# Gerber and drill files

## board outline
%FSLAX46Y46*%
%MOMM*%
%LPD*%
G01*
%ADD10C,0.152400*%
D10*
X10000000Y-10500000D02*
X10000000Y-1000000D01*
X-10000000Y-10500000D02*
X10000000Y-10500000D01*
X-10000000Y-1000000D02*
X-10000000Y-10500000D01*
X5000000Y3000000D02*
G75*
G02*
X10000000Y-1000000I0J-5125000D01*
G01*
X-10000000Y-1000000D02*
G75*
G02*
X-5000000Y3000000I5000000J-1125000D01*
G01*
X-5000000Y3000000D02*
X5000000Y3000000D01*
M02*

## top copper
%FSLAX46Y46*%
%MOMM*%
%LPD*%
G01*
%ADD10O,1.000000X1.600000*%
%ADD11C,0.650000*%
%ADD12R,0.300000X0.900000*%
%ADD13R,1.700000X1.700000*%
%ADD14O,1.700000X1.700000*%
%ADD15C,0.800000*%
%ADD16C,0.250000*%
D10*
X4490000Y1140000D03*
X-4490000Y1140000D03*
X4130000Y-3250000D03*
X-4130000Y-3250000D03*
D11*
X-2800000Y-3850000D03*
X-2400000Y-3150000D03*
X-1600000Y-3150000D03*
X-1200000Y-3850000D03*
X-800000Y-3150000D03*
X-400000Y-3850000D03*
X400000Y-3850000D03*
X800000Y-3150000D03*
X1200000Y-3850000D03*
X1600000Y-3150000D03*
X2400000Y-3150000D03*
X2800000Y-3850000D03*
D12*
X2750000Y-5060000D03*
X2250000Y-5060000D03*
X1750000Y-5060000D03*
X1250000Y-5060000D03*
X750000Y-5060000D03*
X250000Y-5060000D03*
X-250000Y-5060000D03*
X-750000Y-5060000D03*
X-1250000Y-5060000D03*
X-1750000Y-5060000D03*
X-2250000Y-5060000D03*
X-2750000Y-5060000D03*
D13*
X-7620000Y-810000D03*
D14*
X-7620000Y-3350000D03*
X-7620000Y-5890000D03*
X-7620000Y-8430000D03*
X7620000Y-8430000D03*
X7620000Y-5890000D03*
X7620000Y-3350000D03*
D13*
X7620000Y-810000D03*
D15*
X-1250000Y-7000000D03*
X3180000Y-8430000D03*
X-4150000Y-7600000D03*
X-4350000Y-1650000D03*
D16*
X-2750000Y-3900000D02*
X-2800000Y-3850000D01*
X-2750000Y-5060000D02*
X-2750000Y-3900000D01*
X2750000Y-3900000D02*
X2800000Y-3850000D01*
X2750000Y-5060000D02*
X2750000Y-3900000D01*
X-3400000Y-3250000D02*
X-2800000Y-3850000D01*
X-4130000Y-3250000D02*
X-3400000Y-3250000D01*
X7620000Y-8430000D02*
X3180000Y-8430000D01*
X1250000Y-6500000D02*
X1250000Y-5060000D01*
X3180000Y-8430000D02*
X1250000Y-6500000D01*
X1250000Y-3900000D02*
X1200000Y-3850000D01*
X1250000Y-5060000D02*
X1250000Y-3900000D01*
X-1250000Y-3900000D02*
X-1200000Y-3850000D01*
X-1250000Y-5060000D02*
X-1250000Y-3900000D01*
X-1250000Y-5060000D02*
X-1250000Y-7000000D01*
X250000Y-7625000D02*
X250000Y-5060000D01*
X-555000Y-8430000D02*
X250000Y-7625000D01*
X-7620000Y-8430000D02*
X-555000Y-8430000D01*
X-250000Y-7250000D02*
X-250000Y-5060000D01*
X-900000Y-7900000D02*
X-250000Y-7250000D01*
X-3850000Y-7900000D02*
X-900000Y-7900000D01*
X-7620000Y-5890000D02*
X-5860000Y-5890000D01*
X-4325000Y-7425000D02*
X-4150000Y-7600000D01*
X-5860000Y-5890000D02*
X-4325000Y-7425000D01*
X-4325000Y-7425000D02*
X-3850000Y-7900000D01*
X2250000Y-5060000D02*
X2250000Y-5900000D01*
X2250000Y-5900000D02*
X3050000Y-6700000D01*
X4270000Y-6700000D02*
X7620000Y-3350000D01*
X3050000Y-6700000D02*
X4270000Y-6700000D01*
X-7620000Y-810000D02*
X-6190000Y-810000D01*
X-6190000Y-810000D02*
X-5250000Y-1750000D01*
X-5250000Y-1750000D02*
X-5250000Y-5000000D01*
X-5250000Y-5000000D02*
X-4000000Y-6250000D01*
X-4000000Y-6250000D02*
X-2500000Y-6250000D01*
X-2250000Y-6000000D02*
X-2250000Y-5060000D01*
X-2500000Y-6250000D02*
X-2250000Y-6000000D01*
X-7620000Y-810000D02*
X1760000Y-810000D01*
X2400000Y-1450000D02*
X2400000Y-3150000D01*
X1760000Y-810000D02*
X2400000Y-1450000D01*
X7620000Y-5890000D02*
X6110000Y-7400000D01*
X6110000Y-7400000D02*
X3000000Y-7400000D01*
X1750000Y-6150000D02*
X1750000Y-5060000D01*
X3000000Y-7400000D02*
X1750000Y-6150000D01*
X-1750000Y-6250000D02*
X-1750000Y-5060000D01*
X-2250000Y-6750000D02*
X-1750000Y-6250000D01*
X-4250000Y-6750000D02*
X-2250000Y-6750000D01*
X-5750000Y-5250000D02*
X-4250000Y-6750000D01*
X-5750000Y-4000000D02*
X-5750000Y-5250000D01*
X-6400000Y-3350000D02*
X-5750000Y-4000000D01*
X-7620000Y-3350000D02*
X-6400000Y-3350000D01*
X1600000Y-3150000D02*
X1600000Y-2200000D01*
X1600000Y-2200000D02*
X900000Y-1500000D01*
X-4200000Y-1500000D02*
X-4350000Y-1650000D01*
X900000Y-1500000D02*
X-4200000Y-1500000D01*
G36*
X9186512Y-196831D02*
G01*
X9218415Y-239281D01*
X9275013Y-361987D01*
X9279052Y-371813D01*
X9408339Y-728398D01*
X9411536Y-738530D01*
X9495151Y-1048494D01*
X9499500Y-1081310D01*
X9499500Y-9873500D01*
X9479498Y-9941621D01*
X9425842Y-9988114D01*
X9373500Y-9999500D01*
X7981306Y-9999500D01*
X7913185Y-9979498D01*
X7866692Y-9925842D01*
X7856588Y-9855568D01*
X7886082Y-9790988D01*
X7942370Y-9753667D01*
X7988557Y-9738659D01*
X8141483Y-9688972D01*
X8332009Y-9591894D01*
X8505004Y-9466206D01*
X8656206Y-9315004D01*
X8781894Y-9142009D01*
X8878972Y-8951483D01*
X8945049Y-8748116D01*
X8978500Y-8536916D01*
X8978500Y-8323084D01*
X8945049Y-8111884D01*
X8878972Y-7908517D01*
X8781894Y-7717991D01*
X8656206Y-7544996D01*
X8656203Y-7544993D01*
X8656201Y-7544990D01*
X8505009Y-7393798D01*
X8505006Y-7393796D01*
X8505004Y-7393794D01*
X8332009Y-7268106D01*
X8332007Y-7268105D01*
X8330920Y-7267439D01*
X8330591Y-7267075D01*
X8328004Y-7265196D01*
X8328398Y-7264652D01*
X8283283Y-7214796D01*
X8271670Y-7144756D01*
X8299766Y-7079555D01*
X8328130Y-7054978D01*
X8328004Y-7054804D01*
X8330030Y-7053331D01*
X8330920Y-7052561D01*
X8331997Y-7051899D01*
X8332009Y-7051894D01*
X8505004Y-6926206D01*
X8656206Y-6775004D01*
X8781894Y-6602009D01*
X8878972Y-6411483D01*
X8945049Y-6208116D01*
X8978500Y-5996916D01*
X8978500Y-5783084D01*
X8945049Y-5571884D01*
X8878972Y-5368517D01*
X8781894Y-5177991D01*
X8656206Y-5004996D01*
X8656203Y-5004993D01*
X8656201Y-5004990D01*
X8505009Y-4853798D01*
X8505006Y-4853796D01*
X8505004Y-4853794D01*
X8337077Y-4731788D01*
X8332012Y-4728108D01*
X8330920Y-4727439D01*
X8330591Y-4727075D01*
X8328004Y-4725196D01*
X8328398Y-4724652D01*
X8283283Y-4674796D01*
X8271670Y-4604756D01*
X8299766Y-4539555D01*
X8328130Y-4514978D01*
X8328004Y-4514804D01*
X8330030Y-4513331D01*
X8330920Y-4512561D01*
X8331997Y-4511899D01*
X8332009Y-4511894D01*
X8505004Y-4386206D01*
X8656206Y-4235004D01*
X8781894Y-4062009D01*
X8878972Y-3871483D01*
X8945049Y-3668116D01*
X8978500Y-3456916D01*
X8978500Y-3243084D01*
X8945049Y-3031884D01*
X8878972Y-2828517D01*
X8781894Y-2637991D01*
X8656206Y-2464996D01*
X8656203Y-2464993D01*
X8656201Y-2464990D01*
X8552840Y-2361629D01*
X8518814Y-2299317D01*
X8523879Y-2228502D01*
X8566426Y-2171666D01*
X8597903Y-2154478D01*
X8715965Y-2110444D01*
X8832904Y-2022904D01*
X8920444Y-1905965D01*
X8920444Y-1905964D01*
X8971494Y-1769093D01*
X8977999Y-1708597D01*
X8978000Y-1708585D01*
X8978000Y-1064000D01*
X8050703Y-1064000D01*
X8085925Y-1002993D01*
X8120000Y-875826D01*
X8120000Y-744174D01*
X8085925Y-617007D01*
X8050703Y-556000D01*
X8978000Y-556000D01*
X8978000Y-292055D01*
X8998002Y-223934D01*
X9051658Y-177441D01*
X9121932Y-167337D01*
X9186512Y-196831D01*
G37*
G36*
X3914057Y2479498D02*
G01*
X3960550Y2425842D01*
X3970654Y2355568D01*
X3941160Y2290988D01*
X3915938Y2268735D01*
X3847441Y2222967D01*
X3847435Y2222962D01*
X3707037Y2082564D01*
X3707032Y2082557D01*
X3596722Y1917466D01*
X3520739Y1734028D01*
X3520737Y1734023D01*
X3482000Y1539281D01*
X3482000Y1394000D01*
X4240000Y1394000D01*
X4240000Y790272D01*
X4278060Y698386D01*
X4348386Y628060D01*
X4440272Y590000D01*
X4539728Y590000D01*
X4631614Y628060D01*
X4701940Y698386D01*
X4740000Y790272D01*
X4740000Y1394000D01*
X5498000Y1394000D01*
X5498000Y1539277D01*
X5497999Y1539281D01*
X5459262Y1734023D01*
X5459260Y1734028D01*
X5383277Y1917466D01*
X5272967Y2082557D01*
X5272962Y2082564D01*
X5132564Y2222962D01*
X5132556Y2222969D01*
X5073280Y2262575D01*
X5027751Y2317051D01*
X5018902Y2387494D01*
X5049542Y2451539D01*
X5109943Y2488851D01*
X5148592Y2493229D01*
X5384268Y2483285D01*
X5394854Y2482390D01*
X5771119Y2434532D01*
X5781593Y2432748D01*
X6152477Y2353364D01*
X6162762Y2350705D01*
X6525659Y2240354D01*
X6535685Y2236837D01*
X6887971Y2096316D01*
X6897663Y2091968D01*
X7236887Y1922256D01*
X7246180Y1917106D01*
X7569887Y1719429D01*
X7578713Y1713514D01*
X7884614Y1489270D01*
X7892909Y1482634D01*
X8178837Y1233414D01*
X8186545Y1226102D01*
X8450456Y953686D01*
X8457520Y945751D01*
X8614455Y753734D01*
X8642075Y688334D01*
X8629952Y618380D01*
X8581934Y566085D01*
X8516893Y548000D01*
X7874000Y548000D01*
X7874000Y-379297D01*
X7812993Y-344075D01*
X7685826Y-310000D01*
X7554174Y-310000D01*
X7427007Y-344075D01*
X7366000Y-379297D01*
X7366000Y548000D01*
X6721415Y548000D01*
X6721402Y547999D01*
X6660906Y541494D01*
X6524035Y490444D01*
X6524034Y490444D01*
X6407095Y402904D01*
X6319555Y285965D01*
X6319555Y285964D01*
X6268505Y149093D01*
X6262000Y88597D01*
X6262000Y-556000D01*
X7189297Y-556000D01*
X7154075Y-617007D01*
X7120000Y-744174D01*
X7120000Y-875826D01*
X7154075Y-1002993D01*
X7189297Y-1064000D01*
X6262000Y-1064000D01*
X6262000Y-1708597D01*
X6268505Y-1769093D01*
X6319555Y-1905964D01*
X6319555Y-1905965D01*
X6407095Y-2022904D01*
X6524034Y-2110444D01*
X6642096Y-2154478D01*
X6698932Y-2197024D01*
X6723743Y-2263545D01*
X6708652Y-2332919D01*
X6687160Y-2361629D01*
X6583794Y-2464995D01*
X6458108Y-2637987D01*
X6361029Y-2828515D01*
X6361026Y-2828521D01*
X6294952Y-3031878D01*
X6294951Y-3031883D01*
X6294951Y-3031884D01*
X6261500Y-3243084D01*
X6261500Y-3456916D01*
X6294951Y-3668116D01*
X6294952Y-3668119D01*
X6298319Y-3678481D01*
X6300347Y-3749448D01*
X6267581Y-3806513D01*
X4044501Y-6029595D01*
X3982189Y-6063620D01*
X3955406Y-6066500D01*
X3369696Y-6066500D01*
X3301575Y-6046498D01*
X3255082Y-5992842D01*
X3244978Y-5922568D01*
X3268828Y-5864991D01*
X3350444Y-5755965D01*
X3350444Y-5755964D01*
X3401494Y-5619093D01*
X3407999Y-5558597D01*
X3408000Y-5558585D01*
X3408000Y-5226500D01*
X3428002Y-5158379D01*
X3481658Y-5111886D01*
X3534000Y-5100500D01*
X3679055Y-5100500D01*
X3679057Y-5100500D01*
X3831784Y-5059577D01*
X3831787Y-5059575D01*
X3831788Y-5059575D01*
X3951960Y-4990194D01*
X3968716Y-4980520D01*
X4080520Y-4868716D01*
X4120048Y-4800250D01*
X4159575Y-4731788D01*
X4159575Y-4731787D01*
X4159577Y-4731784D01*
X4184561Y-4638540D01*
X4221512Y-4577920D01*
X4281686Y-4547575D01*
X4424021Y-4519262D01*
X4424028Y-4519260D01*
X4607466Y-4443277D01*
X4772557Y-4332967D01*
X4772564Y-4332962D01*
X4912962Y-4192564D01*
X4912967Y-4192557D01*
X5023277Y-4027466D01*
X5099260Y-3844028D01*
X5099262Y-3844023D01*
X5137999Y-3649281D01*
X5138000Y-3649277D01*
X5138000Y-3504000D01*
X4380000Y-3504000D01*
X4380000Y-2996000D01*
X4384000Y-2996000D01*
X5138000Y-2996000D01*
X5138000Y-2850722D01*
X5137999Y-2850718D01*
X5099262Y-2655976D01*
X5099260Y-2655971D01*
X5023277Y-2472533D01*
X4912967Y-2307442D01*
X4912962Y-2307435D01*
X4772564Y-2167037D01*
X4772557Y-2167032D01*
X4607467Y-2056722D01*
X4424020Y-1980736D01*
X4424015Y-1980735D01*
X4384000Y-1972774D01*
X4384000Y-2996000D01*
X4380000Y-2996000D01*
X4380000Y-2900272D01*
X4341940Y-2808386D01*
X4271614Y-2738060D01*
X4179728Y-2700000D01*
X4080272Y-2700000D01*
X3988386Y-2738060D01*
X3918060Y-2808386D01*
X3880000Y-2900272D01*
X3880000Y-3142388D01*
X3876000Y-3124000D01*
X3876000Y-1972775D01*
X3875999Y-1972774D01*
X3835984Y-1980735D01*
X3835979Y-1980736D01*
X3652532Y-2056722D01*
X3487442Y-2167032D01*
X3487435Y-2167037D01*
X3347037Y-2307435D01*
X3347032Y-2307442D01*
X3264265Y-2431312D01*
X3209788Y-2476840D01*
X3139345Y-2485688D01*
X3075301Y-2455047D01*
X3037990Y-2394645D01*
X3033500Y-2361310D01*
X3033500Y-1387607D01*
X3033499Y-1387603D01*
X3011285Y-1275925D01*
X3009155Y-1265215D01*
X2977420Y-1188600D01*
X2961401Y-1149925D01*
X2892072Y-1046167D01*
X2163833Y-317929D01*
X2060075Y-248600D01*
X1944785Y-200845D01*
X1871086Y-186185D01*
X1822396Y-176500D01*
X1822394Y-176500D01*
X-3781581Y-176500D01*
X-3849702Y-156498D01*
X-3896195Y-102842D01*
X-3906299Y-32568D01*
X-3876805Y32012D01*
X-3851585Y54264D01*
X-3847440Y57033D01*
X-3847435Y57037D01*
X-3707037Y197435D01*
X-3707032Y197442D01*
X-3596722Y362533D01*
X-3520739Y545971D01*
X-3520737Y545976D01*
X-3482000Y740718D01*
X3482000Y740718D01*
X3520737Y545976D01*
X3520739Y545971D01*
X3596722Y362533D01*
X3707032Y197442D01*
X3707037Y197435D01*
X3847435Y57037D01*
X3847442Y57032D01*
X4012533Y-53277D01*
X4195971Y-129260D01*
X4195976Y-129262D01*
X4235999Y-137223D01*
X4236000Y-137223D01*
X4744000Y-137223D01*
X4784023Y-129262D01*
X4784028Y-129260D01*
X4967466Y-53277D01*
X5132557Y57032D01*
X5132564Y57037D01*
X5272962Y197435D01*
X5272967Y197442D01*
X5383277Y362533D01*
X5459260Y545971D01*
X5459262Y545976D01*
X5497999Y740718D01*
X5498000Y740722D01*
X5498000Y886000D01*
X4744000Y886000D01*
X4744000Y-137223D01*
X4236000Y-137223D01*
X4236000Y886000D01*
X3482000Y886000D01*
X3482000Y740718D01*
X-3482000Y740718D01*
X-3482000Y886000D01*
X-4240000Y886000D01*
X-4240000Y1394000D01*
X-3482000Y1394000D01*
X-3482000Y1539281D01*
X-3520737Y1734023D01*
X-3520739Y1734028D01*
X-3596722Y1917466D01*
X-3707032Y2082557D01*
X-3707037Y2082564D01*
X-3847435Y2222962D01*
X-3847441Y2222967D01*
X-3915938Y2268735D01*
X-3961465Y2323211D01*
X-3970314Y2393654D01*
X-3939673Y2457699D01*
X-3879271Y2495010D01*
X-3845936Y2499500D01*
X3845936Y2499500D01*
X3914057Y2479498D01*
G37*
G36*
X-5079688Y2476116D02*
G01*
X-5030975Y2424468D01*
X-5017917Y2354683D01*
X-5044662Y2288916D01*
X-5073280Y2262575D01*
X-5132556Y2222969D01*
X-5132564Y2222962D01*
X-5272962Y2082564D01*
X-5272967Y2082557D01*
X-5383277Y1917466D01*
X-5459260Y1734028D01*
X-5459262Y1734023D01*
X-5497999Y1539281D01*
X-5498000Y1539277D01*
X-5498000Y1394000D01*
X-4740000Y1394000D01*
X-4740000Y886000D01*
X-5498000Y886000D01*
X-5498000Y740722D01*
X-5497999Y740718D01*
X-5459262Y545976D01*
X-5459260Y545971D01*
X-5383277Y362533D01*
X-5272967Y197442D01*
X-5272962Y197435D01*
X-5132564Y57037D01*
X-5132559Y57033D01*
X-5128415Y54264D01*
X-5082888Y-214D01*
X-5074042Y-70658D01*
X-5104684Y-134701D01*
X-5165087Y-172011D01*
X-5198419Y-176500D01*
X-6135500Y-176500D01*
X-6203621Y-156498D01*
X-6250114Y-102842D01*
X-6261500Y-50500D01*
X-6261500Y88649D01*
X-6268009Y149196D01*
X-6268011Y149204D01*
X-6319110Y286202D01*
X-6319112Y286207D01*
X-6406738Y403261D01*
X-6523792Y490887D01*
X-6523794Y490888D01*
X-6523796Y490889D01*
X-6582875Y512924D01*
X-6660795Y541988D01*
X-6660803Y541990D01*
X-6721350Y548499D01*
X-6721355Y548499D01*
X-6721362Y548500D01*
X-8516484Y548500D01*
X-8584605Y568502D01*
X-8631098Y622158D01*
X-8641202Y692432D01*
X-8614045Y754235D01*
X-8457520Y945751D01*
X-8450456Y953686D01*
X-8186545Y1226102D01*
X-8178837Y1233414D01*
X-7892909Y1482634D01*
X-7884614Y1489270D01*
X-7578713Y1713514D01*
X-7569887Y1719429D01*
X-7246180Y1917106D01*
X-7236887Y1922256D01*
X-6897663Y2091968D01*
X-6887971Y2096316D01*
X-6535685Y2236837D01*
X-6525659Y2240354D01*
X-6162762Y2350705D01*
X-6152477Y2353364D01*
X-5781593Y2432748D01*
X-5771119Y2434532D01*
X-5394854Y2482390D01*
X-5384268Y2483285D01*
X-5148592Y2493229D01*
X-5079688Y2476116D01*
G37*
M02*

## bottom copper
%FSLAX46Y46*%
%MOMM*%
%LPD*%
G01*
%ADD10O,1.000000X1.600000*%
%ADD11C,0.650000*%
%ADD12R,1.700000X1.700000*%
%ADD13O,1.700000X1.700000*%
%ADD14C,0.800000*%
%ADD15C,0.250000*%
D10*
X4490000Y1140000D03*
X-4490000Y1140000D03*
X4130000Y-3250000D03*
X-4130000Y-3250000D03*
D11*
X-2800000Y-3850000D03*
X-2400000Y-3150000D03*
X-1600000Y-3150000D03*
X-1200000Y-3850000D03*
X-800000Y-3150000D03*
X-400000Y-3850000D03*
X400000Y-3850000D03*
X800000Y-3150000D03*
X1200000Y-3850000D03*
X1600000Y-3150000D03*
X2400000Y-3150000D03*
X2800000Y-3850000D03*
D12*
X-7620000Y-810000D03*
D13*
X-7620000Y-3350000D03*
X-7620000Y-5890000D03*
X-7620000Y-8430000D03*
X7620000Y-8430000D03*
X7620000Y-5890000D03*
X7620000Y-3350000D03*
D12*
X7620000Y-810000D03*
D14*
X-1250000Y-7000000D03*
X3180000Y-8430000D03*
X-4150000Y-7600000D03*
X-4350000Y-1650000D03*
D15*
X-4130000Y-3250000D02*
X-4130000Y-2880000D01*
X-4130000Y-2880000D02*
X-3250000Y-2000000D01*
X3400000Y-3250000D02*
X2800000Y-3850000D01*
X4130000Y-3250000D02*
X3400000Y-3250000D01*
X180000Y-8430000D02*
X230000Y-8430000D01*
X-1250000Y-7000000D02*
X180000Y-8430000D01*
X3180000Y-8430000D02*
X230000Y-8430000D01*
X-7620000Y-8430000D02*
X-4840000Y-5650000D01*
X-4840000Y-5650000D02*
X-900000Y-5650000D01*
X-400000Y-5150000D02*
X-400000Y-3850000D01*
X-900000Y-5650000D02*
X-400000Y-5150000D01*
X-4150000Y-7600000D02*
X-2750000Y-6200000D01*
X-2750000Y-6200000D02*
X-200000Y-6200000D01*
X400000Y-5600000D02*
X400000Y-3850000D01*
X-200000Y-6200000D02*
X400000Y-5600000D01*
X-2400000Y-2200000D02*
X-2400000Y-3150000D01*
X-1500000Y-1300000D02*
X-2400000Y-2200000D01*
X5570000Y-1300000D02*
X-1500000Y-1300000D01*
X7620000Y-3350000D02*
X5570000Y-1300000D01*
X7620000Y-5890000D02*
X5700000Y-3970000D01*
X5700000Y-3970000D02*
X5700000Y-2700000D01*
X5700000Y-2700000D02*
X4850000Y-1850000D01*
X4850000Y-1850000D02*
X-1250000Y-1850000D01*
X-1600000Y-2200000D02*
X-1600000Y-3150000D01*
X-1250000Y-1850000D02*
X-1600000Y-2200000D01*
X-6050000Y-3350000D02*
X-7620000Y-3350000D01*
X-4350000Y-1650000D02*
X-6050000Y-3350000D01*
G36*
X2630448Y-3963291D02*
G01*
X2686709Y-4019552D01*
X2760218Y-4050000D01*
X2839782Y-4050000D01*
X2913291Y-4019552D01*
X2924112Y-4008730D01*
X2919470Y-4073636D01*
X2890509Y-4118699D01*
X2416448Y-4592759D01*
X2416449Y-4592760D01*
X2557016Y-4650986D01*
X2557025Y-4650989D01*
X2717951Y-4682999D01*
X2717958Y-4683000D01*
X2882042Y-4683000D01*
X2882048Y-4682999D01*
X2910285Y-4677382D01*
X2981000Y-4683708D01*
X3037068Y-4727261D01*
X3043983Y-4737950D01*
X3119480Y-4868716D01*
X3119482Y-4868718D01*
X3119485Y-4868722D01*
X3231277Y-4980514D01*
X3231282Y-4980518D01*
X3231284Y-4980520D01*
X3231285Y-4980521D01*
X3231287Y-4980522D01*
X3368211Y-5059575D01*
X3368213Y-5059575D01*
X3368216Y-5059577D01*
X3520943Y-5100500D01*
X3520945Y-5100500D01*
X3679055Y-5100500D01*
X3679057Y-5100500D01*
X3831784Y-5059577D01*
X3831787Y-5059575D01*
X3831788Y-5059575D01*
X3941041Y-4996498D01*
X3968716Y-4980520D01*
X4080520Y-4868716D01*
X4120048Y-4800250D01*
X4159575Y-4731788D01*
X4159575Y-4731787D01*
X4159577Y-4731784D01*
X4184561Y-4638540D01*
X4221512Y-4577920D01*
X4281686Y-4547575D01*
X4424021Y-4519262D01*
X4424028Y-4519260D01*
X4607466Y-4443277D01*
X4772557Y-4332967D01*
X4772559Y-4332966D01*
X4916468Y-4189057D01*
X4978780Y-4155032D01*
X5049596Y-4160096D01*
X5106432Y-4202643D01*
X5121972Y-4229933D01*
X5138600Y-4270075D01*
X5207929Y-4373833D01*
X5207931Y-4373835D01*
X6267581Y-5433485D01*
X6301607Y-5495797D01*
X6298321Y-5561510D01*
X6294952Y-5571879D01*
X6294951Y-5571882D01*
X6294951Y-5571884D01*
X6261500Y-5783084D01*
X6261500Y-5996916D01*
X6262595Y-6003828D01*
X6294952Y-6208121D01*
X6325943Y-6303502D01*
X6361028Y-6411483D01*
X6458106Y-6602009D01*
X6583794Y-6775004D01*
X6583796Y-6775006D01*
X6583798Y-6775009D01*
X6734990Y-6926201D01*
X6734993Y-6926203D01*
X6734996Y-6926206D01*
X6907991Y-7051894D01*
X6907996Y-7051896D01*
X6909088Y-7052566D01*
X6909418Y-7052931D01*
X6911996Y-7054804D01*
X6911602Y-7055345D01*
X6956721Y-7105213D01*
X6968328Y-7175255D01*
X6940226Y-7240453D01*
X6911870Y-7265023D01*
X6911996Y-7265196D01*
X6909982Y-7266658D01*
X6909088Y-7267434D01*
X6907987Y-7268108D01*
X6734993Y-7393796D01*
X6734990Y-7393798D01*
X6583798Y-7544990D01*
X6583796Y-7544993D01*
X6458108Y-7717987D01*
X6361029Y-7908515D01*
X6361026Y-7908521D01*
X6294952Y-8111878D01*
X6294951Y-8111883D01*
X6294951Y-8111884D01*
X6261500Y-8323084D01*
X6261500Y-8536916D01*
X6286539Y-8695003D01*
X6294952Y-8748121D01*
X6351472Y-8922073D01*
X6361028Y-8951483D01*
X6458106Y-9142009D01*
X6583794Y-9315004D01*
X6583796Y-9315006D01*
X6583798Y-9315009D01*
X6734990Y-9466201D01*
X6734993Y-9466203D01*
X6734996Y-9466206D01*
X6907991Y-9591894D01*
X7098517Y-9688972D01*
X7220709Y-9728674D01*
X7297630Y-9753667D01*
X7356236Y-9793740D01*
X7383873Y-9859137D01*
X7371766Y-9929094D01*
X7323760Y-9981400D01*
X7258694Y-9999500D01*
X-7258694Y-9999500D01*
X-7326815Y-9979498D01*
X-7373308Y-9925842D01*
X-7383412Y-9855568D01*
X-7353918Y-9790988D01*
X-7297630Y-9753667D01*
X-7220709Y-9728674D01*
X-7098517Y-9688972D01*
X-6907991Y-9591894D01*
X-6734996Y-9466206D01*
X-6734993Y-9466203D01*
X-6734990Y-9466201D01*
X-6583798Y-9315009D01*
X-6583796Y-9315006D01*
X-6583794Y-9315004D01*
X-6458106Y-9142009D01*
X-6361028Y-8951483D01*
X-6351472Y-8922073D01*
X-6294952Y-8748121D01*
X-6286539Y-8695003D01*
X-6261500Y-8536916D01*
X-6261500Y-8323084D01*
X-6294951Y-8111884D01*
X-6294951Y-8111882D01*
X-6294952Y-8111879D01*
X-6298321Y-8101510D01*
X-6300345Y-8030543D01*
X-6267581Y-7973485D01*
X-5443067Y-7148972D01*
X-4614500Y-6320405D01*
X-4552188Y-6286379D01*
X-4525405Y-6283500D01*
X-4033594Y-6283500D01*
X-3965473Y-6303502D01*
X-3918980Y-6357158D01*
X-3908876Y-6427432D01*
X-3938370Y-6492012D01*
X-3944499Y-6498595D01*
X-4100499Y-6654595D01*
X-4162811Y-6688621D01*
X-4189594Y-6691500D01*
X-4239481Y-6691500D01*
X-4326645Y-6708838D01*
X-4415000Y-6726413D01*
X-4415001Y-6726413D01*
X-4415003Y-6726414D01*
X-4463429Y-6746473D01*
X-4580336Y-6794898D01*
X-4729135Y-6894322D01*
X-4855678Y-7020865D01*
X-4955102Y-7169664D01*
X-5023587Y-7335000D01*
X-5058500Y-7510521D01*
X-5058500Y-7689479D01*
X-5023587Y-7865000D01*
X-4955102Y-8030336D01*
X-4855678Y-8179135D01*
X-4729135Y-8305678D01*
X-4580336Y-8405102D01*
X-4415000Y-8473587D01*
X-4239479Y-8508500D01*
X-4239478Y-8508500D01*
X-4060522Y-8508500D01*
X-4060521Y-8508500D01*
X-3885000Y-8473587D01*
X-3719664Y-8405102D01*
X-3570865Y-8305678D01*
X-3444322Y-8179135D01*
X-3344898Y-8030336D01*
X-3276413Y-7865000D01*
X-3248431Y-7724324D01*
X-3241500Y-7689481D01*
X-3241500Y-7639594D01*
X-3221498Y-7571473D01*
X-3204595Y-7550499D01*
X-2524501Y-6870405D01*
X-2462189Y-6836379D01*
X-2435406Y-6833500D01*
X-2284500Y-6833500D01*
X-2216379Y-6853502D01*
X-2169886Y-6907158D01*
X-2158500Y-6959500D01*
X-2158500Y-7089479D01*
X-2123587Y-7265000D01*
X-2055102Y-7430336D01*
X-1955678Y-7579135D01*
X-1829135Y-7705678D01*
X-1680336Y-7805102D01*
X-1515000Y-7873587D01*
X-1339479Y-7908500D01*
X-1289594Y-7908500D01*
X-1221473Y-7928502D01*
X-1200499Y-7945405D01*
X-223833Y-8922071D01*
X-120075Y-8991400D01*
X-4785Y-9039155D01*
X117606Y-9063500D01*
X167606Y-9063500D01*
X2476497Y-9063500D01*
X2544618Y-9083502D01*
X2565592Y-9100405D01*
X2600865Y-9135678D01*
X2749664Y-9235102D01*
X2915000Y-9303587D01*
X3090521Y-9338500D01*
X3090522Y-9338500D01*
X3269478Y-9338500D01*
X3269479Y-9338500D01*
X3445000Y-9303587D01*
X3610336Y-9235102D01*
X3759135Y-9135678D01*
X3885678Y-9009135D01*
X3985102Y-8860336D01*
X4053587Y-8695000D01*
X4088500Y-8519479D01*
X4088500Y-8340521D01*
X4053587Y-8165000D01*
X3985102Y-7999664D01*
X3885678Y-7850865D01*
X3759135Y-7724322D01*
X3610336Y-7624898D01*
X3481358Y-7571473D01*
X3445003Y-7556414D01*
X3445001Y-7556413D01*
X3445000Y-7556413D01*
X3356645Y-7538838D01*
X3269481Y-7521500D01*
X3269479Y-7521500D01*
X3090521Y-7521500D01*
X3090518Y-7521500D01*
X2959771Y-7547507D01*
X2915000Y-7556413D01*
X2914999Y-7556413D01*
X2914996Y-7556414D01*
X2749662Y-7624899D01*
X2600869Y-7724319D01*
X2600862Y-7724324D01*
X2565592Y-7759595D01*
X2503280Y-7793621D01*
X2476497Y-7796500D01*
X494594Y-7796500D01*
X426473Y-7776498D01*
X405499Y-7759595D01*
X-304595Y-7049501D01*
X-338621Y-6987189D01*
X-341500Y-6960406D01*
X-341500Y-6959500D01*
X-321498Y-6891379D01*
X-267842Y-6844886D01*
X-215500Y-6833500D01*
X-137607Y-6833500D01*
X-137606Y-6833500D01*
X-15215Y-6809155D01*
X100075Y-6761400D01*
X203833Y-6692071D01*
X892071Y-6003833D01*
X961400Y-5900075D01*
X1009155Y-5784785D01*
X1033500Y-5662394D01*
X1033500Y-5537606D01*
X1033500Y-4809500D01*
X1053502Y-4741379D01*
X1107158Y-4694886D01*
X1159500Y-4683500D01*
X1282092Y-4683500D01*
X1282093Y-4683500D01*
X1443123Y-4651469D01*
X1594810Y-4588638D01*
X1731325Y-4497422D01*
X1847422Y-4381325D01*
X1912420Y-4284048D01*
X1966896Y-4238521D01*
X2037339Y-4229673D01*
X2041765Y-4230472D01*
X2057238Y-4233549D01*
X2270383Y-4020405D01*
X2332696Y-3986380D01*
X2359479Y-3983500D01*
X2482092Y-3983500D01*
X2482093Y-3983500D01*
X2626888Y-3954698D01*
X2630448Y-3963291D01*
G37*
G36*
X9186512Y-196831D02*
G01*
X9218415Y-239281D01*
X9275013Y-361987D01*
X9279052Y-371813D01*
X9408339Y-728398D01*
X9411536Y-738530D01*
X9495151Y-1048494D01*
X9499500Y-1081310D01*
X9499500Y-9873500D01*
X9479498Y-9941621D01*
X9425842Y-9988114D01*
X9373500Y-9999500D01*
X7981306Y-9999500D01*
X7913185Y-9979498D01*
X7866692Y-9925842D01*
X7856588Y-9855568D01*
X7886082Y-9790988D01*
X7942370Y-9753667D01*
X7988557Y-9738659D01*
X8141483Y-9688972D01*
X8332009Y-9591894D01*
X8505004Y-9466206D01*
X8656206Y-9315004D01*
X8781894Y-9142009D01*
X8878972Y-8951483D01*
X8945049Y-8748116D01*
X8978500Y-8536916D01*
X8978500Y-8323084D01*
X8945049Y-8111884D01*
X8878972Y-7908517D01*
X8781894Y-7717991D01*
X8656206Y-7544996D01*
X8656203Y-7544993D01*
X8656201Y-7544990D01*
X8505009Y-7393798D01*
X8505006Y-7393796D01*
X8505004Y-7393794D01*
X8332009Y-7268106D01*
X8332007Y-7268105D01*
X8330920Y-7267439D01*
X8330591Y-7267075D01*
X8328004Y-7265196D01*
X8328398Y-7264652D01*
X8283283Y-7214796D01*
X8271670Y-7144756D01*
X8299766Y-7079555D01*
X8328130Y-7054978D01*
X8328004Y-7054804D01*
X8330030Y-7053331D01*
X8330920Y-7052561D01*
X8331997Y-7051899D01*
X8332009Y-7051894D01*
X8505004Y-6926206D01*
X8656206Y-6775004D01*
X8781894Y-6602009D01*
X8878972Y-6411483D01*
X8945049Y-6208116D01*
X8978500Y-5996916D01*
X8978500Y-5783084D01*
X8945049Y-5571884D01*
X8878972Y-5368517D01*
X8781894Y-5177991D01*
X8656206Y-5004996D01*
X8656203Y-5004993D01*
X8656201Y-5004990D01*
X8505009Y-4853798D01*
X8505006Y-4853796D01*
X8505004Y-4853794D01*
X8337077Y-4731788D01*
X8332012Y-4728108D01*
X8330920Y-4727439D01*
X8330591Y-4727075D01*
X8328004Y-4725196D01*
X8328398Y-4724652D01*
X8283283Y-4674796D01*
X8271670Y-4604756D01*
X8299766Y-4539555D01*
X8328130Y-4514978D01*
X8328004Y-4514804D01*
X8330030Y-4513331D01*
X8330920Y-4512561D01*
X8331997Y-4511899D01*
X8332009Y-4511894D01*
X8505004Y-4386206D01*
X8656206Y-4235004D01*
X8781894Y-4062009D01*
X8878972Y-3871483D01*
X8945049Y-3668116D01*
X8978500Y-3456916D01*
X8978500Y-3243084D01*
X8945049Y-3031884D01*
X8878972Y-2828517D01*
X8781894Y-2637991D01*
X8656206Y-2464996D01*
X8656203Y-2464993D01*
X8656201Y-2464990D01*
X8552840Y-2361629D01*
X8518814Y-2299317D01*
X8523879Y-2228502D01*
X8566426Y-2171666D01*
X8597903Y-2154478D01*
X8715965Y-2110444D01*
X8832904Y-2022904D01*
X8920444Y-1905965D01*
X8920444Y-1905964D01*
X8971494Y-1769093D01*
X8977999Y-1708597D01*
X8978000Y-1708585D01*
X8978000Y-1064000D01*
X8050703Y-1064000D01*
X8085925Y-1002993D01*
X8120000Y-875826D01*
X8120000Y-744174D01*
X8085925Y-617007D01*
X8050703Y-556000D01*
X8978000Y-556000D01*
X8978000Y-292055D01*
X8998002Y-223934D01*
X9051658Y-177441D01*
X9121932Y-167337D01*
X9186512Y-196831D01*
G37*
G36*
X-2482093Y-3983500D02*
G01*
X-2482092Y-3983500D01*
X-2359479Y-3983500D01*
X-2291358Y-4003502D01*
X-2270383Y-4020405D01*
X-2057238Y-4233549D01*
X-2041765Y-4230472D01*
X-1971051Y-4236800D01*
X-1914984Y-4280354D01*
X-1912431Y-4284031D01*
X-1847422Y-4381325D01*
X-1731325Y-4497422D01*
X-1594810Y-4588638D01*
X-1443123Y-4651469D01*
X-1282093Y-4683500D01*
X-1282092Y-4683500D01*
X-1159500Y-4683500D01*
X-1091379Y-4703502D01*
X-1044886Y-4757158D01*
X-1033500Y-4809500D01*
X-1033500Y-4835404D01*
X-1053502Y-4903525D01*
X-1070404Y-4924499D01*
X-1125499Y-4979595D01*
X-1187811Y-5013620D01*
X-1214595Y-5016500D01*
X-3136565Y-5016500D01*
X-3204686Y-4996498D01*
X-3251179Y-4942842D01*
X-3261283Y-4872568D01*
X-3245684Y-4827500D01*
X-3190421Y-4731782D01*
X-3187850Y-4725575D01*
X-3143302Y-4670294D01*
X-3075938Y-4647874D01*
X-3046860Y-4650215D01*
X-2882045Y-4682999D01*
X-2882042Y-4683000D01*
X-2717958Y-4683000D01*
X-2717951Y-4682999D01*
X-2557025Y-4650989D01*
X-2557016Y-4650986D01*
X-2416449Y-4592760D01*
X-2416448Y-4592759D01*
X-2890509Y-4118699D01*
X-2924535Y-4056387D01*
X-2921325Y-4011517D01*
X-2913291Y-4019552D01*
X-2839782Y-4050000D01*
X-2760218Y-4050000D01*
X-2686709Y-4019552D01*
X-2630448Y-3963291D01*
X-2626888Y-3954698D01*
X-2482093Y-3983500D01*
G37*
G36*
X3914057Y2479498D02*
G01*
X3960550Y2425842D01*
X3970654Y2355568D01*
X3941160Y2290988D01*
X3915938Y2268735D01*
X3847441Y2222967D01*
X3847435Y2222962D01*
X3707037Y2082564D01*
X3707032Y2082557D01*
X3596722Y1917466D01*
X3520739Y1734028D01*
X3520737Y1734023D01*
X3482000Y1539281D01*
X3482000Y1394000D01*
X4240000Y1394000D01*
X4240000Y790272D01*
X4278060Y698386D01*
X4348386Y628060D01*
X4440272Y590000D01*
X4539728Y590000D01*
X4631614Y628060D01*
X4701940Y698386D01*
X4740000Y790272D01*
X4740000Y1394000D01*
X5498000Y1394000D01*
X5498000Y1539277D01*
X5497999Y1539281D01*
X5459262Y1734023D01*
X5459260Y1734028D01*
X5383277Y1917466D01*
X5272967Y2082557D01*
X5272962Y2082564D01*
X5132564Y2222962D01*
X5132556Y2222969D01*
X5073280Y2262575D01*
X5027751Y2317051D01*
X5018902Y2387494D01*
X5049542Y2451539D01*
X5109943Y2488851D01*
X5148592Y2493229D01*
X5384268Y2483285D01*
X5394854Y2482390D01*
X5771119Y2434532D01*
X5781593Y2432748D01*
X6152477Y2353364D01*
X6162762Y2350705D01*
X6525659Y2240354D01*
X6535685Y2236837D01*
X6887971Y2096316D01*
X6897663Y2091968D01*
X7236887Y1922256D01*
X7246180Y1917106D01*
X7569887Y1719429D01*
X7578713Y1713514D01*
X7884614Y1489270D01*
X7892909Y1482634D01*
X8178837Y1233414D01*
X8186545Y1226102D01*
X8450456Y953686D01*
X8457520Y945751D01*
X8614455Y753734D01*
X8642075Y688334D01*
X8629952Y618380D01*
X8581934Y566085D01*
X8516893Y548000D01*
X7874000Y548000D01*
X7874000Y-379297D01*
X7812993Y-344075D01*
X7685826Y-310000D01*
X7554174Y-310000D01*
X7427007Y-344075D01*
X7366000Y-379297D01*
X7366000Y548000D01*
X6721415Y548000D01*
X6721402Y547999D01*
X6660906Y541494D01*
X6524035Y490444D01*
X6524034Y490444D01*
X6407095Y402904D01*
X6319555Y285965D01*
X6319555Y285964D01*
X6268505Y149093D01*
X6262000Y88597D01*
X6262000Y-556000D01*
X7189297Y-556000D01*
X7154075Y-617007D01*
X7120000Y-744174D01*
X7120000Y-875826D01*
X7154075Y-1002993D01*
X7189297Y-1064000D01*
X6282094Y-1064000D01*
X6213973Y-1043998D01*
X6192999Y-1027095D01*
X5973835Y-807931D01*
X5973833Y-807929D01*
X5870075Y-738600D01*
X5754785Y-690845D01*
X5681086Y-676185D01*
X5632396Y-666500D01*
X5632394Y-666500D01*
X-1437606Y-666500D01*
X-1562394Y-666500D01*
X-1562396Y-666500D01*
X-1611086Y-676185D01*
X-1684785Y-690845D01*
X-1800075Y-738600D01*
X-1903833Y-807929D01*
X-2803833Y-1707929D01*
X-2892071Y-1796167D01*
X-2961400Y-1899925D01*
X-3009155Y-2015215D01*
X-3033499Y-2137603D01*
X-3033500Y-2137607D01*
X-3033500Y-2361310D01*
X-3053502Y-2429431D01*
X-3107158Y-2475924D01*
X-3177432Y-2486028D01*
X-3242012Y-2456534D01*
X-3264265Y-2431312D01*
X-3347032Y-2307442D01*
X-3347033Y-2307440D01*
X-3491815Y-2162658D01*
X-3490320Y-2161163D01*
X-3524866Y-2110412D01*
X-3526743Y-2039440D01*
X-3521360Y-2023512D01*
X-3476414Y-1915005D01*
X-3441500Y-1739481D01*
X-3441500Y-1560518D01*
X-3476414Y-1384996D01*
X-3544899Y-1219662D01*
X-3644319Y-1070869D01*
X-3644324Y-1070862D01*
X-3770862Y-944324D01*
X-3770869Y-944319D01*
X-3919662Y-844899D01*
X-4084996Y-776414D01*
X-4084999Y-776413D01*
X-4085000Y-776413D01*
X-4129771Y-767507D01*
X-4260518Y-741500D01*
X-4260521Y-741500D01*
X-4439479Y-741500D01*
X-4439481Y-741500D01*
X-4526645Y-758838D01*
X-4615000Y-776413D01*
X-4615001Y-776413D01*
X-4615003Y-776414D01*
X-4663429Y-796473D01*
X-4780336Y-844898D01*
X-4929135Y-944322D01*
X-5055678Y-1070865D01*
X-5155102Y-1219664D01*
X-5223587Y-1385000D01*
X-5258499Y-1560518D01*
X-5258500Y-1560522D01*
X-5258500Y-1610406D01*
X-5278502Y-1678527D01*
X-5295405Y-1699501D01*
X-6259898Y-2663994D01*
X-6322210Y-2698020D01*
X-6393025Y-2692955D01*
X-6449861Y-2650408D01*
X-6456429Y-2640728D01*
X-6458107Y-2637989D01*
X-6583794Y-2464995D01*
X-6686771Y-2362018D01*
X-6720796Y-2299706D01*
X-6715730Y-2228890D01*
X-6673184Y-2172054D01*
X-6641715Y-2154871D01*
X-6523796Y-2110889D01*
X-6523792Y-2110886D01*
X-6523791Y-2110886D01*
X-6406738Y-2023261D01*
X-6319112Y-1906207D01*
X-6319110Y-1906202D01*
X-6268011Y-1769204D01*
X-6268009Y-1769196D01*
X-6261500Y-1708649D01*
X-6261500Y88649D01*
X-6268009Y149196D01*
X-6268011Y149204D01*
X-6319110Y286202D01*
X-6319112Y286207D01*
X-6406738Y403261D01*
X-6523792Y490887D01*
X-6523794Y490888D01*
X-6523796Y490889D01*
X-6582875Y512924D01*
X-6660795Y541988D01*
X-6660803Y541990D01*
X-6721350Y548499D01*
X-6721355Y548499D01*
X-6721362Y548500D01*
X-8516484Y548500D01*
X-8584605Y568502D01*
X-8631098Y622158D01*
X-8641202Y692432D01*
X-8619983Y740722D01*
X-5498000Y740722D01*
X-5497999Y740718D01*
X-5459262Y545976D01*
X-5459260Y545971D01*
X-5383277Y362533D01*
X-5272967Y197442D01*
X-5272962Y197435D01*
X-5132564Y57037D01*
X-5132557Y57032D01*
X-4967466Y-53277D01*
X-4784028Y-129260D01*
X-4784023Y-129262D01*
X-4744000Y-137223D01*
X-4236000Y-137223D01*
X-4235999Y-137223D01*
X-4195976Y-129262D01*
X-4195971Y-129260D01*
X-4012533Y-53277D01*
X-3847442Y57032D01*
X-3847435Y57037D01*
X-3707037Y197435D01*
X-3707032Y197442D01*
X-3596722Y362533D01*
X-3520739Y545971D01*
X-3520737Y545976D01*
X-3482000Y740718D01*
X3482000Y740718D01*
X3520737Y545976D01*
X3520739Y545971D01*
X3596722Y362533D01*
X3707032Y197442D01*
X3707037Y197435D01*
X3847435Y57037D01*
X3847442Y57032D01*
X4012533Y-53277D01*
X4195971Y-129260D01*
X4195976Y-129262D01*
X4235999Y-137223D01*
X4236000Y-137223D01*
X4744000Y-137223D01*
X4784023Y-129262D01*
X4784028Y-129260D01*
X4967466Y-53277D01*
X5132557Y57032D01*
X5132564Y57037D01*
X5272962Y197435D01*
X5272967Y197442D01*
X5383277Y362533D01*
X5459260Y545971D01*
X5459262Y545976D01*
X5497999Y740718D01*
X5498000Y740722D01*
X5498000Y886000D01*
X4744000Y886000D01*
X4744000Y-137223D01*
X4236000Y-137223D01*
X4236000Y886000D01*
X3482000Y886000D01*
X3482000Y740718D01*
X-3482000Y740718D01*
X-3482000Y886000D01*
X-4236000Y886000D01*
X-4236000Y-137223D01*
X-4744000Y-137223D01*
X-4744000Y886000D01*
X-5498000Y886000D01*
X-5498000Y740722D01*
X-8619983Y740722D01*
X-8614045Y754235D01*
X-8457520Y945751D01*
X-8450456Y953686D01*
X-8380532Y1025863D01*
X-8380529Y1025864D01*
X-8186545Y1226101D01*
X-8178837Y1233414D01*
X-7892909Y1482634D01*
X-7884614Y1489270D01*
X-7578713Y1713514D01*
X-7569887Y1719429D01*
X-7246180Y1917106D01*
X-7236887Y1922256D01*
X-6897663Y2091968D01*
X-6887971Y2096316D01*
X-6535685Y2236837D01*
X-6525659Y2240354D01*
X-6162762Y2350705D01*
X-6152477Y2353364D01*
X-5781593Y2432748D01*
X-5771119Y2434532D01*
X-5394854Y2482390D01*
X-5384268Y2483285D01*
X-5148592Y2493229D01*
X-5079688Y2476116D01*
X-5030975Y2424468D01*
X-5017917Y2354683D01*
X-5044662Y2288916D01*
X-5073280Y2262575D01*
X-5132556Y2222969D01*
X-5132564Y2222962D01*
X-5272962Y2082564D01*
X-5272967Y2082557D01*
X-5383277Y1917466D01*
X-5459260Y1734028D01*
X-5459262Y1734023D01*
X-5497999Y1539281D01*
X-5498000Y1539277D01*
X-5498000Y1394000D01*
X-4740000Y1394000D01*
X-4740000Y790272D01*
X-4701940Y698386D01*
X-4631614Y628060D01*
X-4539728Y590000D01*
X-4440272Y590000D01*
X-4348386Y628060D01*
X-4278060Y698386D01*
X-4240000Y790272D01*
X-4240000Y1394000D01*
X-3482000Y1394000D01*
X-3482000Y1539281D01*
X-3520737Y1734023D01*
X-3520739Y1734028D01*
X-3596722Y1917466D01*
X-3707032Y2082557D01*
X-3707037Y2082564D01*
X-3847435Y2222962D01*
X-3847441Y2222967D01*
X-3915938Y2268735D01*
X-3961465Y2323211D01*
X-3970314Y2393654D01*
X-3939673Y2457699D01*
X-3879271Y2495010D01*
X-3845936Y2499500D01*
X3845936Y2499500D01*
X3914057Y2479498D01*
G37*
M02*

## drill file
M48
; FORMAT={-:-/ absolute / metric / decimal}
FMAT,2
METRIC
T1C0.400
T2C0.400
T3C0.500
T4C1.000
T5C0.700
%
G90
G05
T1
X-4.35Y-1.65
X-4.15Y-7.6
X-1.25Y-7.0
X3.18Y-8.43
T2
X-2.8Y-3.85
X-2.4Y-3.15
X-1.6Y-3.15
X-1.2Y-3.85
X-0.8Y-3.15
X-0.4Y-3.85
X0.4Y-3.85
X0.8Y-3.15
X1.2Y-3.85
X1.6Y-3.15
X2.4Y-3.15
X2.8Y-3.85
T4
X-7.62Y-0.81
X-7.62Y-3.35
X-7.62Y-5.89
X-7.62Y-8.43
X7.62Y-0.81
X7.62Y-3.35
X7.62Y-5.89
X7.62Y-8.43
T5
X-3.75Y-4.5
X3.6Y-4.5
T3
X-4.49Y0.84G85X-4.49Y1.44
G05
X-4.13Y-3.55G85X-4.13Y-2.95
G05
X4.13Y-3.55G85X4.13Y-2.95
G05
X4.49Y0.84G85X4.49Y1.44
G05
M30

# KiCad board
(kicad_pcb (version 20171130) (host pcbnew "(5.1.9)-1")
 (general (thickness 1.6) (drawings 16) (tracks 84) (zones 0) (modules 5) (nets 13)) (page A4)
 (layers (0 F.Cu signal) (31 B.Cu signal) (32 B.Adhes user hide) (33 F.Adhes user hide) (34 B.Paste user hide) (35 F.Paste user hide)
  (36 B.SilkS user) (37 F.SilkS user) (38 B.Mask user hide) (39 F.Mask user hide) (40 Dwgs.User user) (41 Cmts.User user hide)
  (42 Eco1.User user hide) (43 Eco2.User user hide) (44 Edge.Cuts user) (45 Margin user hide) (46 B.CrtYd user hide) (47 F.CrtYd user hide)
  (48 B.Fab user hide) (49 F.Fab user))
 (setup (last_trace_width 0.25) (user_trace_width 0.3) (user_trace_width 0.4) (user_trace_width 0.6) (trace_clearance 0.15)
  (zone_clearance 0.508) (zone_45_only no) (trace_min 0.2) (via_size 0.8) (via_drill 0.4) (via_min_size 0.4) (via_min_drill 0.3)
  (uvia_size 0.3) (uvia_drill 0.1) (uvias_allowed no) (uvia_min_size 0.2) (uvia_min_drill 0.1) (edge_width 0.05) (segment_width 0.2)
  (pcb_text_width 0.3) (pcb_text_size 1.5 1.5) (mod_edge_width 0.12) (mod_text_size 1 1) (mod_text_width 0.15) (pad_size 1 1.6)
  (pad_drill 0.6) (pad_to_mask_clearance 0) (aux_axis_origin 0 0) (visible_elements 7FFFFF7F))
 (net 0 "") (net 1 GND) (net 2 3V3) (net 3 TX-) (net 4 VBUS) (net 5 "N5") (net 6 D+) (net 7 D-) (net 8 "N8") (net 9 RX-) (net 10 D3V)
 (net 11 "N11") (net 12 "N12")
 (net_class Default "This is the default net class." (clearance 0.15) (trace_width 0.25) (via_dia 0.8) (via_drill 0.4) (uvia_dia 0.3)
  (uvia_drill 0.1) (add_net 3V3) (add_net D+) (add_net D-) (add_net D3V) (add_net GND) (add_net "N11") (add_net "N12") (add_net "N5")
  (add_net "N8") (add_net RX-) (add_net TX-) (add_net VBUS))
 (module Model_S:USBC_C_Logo (layer F.Cu) (at -0.25 8.25)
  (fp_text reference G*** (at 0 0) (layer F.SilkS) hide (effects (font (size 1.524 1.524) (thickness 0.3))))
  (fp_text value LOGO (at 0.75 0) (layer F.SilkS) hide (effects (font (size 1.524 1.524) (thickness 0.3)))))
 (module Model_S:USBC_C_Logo (layer F.Cu) (at 136.91 121.42)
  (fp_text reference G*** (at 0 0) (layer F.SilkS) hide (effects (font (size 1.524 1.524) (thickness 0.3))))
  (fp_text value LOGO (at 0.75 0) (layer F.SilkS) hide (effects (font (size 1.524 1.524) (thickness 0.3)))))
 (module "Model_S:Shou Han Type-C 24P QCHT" (layer F.Cu) (at 0 -3 180)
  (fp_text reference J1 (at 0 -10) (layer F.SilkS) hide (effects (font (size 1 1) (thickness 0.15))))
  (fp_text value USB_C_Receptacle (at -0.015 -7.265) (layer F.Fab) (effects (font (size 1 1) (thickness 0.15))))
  (pad S1 thru_hole oval (at -4.49 -1.86 180) (size 1 1.6) (drill oval 0.5 1.1) (layers *.Cu *.Mask) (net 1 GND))
  (pad S1 thru_hole oval (at 4.49 -1.86 180) (size 1 1.6) (drill oval 0.5 1.1) (layers *.Cu *.Mask) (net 1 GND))
  (pad S1 thru_hole oval (at -4.13 -6.25 180) (size 1 1.6) (drill oval 0.5 1.1) (layers *.Cu *.Mask) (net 1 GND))
  (pad S1 thru_hole oval (at 4.13 -6.25 180) (size 1 1.6) (drill oval 0.5 1.1) (layers *.Cu *.Mask) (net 1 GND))
  (pad B1 thru_hole circle (at 2.8 -6.85 180) (size 0.65 0.65) (drill 0.4) (layers *.Cu *.Mask) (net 1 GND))
  (pad B2 thru_hole circle (at 2.4 -6.15 180) (size 0.65 0.65) (drill 0.4) (layers *.Cu *.Mask) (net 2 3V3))
  (pad B3 thru_hole circle (at 1.6 -6.15 180) (size 0.65 0.65) (drill 0.4) (layers *.Cu *.Mask) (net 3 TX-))
  (pad B4 thru_hole circle (at 1.2 -6.85 180) (size 0.65 0.65) (drill 0.4) (layers *.Cu *.Mask) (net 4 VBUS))
  (pad B5 thru_hole circle (at 0.8 -6.15 180) (size 0.65 0.65) (drill 0.4) (layers *.Cu *.Mask) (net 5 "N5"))
  (pad B6 thru_hole circle (at 0.4 -6.85 180) (size 0.65 0.65) (drill 0.4) (layers *.Cu *.Mask) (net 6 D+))
  (pad B7 thru_hole circle (at -0.4 -6.85 180) (size 0.65 0.65) (drill 0.4) (layers *.Cu *.Mask) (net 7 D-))
  (pad B8 thru_hole circle (at -0.8 -6.15 180) (size 0.65 0.65) (drill 0.4) (layers *.Cu *.Mask) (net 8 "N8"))
  (pad B9 thru_hole circle (at -1.2 -6.85 180) (size 0.65 0.65) (drill 0.4) (layers *.Cu *.Mask) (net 4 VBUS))
  (pad B10 thru_hole circle (at -1.6 -6.15 180) (size 0.65 0.65) (drill 0.4) (layers *.Cu *.Mask) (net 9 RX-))
  (pad B11 thru_hole circle (at -2.4 -6.15 180) (size 0.65 0.65) (drill 0.4) (layers *.Cu *.Mask) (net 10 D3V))
  (pad B12 thru_hole circle (at -2.8 -6.85 180) (size 0.65 0.65) (drill 0.4) (layers *.Cu *.Mask) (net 1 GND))
  (pad "" np_thru_hole circle (at -3.6 -7.5 180) (size 0.7 0.7) (drill 0.7) (layers *.Cu *.Mask))
  (pad "" np_thru_hole circle (at 3.75 -7.5 180) (size 0.7 0.7) (drill 0.7) (layers *.Cu *.Mask))
  (pad A1 smd rect (at -2.75 -8.06 180) (size 0.3 0.9) (layers F.Cu F.Paste F.Mask) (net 1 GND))
  (pad A2 smd rect (at -2.25 -8.06 180) (size 0.3 0.9) (layers F.Cu F.Paste F.Mask) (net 2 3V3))
  (pad A3 smd rect (at -1.75 -8.06 180) (size 0.3 0.9) (layers F.Cu F.Paste F.Mask) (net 3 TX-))
  (pad A4 smd rect (at -1.25 -8.06 180) (size 0.3 0.9) (layers F.Cu F.Paste F.Mask) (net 4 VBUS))
  (pad A5 smd rect (at -0.75 -8.06 180) (size 0.3 0.9) (layers F.Cu F.Paste F.Mask) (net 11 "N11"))
  (pad A6 smd rect (at -0.25 -8.06 180) (size 0.3 0.9) (layers F.Cu F.Paste F.Mask) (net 6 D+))
  (pad A7 smd rect (at 0.25 -8.06 180) (size 0.3 0.9) (layers F.Cu F.Paste F.Mask) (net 7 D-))
  (pad A8 smd rect (at 0.75 -8.06 180) (size 0.3 0.9) (layers F.Cu F.Paste F.Mask) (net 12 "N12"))
  (pad A9 smd rect (at 1.25 -8.06 180) (size 0.3 0.9) (layers F.Cu F.Paste F.Mask) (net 4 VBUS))
  (pad A10 smd rect (at 1.75 -8.06 180) (size 0.3 0.9) (layers F.Cu F.Paste F.Mask) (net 9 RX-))
  (pad A11 smd rect (at 2.25 -8.06 180) (size 0.3 0.9) (layers F.Cu F.Paste F.Mask) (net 10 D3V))
  (pad A12 smd rect (at 2.75 -8.06 180) (size 0.3 0.9) (layers F.Cu F.Paste F.Mask) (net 1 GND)))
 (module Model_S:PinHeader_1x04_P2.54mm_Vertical (layer F.Cu) (at -7.62 0.81)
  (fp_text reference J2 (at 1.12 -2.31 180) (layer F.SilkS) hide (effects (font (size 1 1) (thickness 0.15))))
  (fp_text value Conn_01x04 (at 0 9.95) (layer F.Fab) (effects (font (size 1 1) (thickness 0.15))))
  (pad 1 thru_hole rect (at 0 0) (size 1.7 1.7) (drill 1) (layers *.Cu *.Mask) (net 10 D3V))
  (pad 2 thru_hole oval (at 0 2.54) (size 1.7 1.7) (drill 1) (layers *.Cu *.Mask) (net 9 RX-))
  (pad 3 thru_hole oval (at 0 5.08) (size 1.7 1.7) (drill 1) (layers *.Cu *.Mask) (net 7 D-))
  (pad 4 thru_hole oval (at 0 7.62) (size 1.7 1.7) (drill 1) (layers *.Cu *.Mask) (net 6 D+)))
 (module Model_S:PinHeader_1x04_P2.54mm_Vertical (layer F.Cu) (at 7.62 0.81)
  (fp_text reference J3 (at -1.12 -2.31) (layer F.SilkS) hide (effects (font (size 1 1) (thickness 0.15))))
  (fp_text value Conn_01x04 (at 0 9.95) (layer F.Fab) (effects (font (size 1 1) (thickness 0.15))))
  (pad 4 thru_hole oval (at 0 7.62) (size 1.7 1.7) (drill 1) (layers *.Cu *.Mask) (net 4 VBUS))
  (pad 3 thru_hole oval (at 0 5.08) (size 1.7 1.7) (drill 1) (layers *.Cu *.Mask) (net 3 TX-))
  (pad 2 thru_hole oval (at 0 2.54) (size 1.7 1.7) (drill 1) (layers *.Cu *.Mask) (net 2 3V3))
  (pad 1 thru_hole rect (at 0 0) (size 1.7 1.7) (drill 1) (layers *.Cu *.Mask) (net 1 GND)))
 (gr_line (start 10 10.5) (end 10 1) (layer Edge.Cuts) (width 0.1524))
 (gr_line (start -10 10.5) (end 10 10.5) (layer Edge.Cuts) (width 0.1524))
 (gr_line (start -10 1) (end -10 10.5) (layer Edge.Cuts) (width 0.1524))
 (gr_arc (start 5 2.125) (end 5 -3) (angle 77.319617) (layer Edge.Cuts) (width 0.1524))
 (gr_arc (start -5 2.125) (end -5 -3) (angle -77.319617) (layer Edge.Cuts) (width 0.1524))
 (gr_line (start -5 -3) (end 5 -3) (layer Edge.Cuts) (width 0.1524))
 (segment (start -4.13 3.25) (end -4.13 2.88) (width 0.25) (layer B.Cu) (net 1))
 (segment (start -4.13 2.88) (end -3.25 2) (width 0.25) (layer B.Cu) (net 1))
 (segment (start -2.75 3.9) (end -2.8 3.85) (width 0.25) (layer F.Cu) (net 1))
 (segment (start -2.75 5.06) (end -2.75 3.9) (width 0.25) (layer F.Cu) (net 1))
 (segment (start 2.75 3.9) (end 2.8 3.85) (width 0.25) (layer F.Cu) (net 1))
 (segment (start 2.75 5.06) (end 2.75 3.9) (width 0.25) (layer F.Cu) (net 1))
 (segment (start -3.4 3.25) (end -2.8 3.85) (width 0.25) (layer F.Cu) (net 1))
 (segment (start -4.13 3.25) (end -3.4 3.25) (width 0.25) (layer F.Cu) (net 1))
 (segment (start 3.4 3.25) (end 2.8 3.85) (width 0.25) (layer B.Cu) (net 1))
 (segment (start 4.13 3.25) (end 3.4 3.25) (width 0.25) (layer B.Cu) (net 1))
 (segment (start 7.62 8.43) (end 3.18 8.43) (width 0.25) (layer F.Cu) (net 4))
 (segment (start 1.25 6.5) (end 1.25 5.06) (width 0.25) (layer F.Cu) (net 4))
 (segment (start 3.18 8.43) (end 1.25 6.5) (width 0.25) (layer F.Cu) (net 4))
 (segment (start 1.25 3.9) (end 1.2 3.85) (width 0.25) (layer F.Cu) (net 4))
 (segment (start 1.25 5.06) (end 1.25 3.9) (width 0.25) (layer F.Cu) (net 4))
 (segment (start -1.25 3.9) (end -1.2 3.85) (width 0.25) (layer F.Cu) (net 4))
 (segment (start -1.25 5.06) (end -1.25 3.9) (width 0.25) (layer F.Cu) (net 4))
 (segment (start -1.25 5.06) (end -1.25 7) (width 0.25) (layer F.Cu) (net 4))
 (via (at -1.25 7) (size 0.8) (drill 0.4) (layers F.Cu B.Cu) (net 4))
 (segment (start 0.18 8.43) (end 0.23 8.43) (width 0.25) (layer B.Cu) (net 4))
 (segment (start -1.25 7) (end 0.18 8.43) (width 0.25) (layer B.Cu) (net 4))
 (segment (start 3.18 8.43) (end 0.23 8.43) (width 0.25) (layer B.Cu) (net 4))
 (via (at 3.18 8.43) (size 0.8) (drill 0.4) (layers F.Cu B.Cu) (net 4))
 (segment (start 0.25 7.625) (end 0.25 5.06) (width 0.25) (layer F.Cu) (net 6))
 (segment (start -0.555 8.43) (end 0.25 7.625) (width 0.25) (layer F.Cu) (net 6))
 (segment (start -7.62 8.43) (end -0.555 8.43) (width 0.25) (layer F.Cu) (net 6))
 (segment (start -7.62 8.43) (end -4.84 5.65) (width 0.25) (layer B.Cu) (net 6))
 (segment (start -4.84 5.65) (end -0.9 5.65) (width 0.25) (layer B.Cu) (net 6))
 (segment (start -0.4 5.15) (end -0.4 3.85) (width 0.25) (layer B.Cu) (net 6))
 (segment (start -0.9 5.65) (end -0.4 5.15) (width 0.25) (layer B.Cu) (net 6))
 (segment (start -0.25 7.25) (end -0.25 5.06) (width 0.25) (layer F.Cu) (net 7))
 (segment (start -0.9 7.9) (end -0.25 7.25) (width 0.25) (layer F.Cu) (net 7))
 (segment (start -3.85 7.9) (end -0.9 7.9) (width 0.25) (layer F.Cu) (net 7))
 (segment (start -7.62 5.89) (end -5.86 5.89) (width 0.25) (layer F.Cu) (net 7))
 (via (at -4.15 7.6) (size 0.8) (drill 0.4) (layers F.Cu B.Cu) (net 7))
 (segment (start -4.325 7.425) (end -4.15 7.6) (width 0.25) (layer F.Cu) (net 7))
 (segment (start -5.86 5.89) (end -4.325 7.425) (width 0.25) (layer F.Cu) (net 7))
 (segment (start -4.325 7.425) (end -3.85 7.9) (width 0.25) (layer F.Cu) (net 7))
 (segment (start -4.15 7.6) (end -2.75 6.2) (width 0.25) (layer B.Cu) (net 7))
 (segment (start -2.75 6.2) (end -0.2 6.2) (width 0.25) (layer B.Cu) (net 7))
 (segment (start 0.4 5.6) (end 0.4 3.85) (width 0.25) (layer B.Cu) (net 7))
 (segment (start -0.2 6.2) (end 0.4 5.6) (width 0.25) (layer B.Cu) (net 7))
 (segment (start 2.25 5.06) (end 2.25 5.9) (width 0.25) (layer F.Cu) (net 2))
 (segment (start 2.25 5.9) (end 3.05 6.7) (width 0.25) (layer F.Cu) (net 2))
 (segment (start 4.27 6.7) (end 7.62 3.35) (width 0.25) (layer F.Cu) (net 2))
 (segment (start 3.05 6.7) (end 4.27 6.7) (width 0.25) (layer F.Cu) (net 2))
 (segment (start -2.4 2.2) (end -2.4 3.15) (width 0.25) (layer B.Cu) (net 2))
 (segment (start -1.5 1.3) (end -2.4 2.2) (width 0.25) (layer B.Cu) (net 2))
 (segment (start 5.57 1.3) (end -1.5 1.3) (width 0.25) (layer B.Cu) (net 2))
 (segment (start 7.62 3.35) (end 5.57 1.3) (width 0.25) (layer B.Cu) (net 2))
 (segment (start -7.62 0.81) (end -6.19 0.81) (width 0.25) (layer F.Cu) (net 10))
 (segment (start -6.19 0.81) (end -5.25 1.75) (width 0.25) (layer F.Cu) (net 10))
 (segment (start -5.25 1.75) (end -5.25 5) (width 0.25) (layer F.Cu) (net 10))
 (segment (start -5.25 5) (end -4 6.25) (width 0.25) (layer F.Cu) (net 10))
 (segment (start -4 6.25) (end -2.5 6.25) (width 0.25) (layer F.Cu) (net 10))
 (segment (start -2.25 6) (end -2.25 5.06) (width 0.25) (layer F.Cu) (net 10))
 (segment (start -2.5 6.25) (end -2.25 6) (width 0.25) (layer F.Cu) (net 10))
 (segment (start -7.62 0.81) (end 1.76 0.81) (width 0.25) (layer F.Cu) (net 10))
 (segment (start 2.4 1.45) (end 2.4 3.15) (width 0.25) (layer F.Cu) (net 10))
 (segment (start 1.76 0.81) (end 2.4 1.45) (width 0.25) (layer F.Cu) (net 10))
 (segment (start 7.62 5.89) (end 6.11 7.4) (width 0.25) (layer F.Cu) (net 3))
 (segment (start 6.11 7.4) (end 3 7.4) (width 0.25) (layer F.Cu) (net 3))
 (segment (start 1.75 6.15) (end 1.75 5.06) (width 0.25) (layer F.Cu) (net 3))
 (segment (start 3 7.4) (end 1.75 6.15) (width 0.25) (layer F.Cu) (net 3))
 (segment (start 7.62 5.89) (end 5.7 3.97) (width 0.25) (layer B.Cu) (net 3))
 (segment (start 5.7 3.97) (end 5.7 2.7) (width 0.25) (layer B.Cu) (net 3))
 (segment (start 5.7 2.7) (end 4.85 1.85) (width 0.25) (layer B.Cu) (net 3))
 (segment (start 4.85 1.85) (end -1.25 1.85) (width 0.25) (layer B.Cu) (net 3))
 (segment (start -1.6 2.2) (end -1.6 3.15) (width 0.25) (layer B.Cu) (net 3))
 (segment (start -1.25 1.85) (end -1.6 2.2) (width 0.25) (layer B.Cu) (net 3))
 (segment (start -1.75 6.25) (end -1.75 5.06) (width 0.25) (layer F.Cu) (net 9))
 (segment (start -2.25 6.75) (end -1.75 6.25) (width 0.25) (layer F.Cu) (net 9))
 (segment (start -4.25 6.75) (end -2.25 6.75) (width 0.25) (layer F.Cu) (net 9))
 (segment (start -5.75 5.25) (end -4.25 6.75) (width 0.25) (layer F.Cu) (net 9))
 (segment (start -5.75 4) (end -5.75 5.25) (width 0.25) (layer F.Cu) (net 9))
 (segment (start -6.4 3.35) (end -5.75 4) (width 0.25) (layer F.Cu) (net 9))
 (segment (start -7.62 3.35) (end -6.4 3.35) (width 0.25) (layer F.Cu) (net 9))
 (segment (start 1.6 3.15) (end 1.6 2.2) (width 0.25) (layer F.Cu) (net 9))
 (segment (start 1.6 2.2) (end 0.9 1.5) (width 0.25) (layer F.Cu) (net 9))
 (via (at -4.35 1.65) (size 0.8) (drill 0.4) (layers F.Cu B.Cu) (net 9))
 (segment (start -4.2 1.5) (end -4.35 1.65) (width 0.25) (layer F.Cu) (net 9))
 (segment (start 0.9 1.5) (end -4.2 1.5) (width 0.25) (layer F.Cu) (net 9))
 (segment (start -6.05 3.35) (end -7.62 3.35) (width 0.25) (layer B.Cu) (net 9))
 (segment (start -4.35 1.65) (end -6.05 3.35) (width 0.25) (layer B.Cu) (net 9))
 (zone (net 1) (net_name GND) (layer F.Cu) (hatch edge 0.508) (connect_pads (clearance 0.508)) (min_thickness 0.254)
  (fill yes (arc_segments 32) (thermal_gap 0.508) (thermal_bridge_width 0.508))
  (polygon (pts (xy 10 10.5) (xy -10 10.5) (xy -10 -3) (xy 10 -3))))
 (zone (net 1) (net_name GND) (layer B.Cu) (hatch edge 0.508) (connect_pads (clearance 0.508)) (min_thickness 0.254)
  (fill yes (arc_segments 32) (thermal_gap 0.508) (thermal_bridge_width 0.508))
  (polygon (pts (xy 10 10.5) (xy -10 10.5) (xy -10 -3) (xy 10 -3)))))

